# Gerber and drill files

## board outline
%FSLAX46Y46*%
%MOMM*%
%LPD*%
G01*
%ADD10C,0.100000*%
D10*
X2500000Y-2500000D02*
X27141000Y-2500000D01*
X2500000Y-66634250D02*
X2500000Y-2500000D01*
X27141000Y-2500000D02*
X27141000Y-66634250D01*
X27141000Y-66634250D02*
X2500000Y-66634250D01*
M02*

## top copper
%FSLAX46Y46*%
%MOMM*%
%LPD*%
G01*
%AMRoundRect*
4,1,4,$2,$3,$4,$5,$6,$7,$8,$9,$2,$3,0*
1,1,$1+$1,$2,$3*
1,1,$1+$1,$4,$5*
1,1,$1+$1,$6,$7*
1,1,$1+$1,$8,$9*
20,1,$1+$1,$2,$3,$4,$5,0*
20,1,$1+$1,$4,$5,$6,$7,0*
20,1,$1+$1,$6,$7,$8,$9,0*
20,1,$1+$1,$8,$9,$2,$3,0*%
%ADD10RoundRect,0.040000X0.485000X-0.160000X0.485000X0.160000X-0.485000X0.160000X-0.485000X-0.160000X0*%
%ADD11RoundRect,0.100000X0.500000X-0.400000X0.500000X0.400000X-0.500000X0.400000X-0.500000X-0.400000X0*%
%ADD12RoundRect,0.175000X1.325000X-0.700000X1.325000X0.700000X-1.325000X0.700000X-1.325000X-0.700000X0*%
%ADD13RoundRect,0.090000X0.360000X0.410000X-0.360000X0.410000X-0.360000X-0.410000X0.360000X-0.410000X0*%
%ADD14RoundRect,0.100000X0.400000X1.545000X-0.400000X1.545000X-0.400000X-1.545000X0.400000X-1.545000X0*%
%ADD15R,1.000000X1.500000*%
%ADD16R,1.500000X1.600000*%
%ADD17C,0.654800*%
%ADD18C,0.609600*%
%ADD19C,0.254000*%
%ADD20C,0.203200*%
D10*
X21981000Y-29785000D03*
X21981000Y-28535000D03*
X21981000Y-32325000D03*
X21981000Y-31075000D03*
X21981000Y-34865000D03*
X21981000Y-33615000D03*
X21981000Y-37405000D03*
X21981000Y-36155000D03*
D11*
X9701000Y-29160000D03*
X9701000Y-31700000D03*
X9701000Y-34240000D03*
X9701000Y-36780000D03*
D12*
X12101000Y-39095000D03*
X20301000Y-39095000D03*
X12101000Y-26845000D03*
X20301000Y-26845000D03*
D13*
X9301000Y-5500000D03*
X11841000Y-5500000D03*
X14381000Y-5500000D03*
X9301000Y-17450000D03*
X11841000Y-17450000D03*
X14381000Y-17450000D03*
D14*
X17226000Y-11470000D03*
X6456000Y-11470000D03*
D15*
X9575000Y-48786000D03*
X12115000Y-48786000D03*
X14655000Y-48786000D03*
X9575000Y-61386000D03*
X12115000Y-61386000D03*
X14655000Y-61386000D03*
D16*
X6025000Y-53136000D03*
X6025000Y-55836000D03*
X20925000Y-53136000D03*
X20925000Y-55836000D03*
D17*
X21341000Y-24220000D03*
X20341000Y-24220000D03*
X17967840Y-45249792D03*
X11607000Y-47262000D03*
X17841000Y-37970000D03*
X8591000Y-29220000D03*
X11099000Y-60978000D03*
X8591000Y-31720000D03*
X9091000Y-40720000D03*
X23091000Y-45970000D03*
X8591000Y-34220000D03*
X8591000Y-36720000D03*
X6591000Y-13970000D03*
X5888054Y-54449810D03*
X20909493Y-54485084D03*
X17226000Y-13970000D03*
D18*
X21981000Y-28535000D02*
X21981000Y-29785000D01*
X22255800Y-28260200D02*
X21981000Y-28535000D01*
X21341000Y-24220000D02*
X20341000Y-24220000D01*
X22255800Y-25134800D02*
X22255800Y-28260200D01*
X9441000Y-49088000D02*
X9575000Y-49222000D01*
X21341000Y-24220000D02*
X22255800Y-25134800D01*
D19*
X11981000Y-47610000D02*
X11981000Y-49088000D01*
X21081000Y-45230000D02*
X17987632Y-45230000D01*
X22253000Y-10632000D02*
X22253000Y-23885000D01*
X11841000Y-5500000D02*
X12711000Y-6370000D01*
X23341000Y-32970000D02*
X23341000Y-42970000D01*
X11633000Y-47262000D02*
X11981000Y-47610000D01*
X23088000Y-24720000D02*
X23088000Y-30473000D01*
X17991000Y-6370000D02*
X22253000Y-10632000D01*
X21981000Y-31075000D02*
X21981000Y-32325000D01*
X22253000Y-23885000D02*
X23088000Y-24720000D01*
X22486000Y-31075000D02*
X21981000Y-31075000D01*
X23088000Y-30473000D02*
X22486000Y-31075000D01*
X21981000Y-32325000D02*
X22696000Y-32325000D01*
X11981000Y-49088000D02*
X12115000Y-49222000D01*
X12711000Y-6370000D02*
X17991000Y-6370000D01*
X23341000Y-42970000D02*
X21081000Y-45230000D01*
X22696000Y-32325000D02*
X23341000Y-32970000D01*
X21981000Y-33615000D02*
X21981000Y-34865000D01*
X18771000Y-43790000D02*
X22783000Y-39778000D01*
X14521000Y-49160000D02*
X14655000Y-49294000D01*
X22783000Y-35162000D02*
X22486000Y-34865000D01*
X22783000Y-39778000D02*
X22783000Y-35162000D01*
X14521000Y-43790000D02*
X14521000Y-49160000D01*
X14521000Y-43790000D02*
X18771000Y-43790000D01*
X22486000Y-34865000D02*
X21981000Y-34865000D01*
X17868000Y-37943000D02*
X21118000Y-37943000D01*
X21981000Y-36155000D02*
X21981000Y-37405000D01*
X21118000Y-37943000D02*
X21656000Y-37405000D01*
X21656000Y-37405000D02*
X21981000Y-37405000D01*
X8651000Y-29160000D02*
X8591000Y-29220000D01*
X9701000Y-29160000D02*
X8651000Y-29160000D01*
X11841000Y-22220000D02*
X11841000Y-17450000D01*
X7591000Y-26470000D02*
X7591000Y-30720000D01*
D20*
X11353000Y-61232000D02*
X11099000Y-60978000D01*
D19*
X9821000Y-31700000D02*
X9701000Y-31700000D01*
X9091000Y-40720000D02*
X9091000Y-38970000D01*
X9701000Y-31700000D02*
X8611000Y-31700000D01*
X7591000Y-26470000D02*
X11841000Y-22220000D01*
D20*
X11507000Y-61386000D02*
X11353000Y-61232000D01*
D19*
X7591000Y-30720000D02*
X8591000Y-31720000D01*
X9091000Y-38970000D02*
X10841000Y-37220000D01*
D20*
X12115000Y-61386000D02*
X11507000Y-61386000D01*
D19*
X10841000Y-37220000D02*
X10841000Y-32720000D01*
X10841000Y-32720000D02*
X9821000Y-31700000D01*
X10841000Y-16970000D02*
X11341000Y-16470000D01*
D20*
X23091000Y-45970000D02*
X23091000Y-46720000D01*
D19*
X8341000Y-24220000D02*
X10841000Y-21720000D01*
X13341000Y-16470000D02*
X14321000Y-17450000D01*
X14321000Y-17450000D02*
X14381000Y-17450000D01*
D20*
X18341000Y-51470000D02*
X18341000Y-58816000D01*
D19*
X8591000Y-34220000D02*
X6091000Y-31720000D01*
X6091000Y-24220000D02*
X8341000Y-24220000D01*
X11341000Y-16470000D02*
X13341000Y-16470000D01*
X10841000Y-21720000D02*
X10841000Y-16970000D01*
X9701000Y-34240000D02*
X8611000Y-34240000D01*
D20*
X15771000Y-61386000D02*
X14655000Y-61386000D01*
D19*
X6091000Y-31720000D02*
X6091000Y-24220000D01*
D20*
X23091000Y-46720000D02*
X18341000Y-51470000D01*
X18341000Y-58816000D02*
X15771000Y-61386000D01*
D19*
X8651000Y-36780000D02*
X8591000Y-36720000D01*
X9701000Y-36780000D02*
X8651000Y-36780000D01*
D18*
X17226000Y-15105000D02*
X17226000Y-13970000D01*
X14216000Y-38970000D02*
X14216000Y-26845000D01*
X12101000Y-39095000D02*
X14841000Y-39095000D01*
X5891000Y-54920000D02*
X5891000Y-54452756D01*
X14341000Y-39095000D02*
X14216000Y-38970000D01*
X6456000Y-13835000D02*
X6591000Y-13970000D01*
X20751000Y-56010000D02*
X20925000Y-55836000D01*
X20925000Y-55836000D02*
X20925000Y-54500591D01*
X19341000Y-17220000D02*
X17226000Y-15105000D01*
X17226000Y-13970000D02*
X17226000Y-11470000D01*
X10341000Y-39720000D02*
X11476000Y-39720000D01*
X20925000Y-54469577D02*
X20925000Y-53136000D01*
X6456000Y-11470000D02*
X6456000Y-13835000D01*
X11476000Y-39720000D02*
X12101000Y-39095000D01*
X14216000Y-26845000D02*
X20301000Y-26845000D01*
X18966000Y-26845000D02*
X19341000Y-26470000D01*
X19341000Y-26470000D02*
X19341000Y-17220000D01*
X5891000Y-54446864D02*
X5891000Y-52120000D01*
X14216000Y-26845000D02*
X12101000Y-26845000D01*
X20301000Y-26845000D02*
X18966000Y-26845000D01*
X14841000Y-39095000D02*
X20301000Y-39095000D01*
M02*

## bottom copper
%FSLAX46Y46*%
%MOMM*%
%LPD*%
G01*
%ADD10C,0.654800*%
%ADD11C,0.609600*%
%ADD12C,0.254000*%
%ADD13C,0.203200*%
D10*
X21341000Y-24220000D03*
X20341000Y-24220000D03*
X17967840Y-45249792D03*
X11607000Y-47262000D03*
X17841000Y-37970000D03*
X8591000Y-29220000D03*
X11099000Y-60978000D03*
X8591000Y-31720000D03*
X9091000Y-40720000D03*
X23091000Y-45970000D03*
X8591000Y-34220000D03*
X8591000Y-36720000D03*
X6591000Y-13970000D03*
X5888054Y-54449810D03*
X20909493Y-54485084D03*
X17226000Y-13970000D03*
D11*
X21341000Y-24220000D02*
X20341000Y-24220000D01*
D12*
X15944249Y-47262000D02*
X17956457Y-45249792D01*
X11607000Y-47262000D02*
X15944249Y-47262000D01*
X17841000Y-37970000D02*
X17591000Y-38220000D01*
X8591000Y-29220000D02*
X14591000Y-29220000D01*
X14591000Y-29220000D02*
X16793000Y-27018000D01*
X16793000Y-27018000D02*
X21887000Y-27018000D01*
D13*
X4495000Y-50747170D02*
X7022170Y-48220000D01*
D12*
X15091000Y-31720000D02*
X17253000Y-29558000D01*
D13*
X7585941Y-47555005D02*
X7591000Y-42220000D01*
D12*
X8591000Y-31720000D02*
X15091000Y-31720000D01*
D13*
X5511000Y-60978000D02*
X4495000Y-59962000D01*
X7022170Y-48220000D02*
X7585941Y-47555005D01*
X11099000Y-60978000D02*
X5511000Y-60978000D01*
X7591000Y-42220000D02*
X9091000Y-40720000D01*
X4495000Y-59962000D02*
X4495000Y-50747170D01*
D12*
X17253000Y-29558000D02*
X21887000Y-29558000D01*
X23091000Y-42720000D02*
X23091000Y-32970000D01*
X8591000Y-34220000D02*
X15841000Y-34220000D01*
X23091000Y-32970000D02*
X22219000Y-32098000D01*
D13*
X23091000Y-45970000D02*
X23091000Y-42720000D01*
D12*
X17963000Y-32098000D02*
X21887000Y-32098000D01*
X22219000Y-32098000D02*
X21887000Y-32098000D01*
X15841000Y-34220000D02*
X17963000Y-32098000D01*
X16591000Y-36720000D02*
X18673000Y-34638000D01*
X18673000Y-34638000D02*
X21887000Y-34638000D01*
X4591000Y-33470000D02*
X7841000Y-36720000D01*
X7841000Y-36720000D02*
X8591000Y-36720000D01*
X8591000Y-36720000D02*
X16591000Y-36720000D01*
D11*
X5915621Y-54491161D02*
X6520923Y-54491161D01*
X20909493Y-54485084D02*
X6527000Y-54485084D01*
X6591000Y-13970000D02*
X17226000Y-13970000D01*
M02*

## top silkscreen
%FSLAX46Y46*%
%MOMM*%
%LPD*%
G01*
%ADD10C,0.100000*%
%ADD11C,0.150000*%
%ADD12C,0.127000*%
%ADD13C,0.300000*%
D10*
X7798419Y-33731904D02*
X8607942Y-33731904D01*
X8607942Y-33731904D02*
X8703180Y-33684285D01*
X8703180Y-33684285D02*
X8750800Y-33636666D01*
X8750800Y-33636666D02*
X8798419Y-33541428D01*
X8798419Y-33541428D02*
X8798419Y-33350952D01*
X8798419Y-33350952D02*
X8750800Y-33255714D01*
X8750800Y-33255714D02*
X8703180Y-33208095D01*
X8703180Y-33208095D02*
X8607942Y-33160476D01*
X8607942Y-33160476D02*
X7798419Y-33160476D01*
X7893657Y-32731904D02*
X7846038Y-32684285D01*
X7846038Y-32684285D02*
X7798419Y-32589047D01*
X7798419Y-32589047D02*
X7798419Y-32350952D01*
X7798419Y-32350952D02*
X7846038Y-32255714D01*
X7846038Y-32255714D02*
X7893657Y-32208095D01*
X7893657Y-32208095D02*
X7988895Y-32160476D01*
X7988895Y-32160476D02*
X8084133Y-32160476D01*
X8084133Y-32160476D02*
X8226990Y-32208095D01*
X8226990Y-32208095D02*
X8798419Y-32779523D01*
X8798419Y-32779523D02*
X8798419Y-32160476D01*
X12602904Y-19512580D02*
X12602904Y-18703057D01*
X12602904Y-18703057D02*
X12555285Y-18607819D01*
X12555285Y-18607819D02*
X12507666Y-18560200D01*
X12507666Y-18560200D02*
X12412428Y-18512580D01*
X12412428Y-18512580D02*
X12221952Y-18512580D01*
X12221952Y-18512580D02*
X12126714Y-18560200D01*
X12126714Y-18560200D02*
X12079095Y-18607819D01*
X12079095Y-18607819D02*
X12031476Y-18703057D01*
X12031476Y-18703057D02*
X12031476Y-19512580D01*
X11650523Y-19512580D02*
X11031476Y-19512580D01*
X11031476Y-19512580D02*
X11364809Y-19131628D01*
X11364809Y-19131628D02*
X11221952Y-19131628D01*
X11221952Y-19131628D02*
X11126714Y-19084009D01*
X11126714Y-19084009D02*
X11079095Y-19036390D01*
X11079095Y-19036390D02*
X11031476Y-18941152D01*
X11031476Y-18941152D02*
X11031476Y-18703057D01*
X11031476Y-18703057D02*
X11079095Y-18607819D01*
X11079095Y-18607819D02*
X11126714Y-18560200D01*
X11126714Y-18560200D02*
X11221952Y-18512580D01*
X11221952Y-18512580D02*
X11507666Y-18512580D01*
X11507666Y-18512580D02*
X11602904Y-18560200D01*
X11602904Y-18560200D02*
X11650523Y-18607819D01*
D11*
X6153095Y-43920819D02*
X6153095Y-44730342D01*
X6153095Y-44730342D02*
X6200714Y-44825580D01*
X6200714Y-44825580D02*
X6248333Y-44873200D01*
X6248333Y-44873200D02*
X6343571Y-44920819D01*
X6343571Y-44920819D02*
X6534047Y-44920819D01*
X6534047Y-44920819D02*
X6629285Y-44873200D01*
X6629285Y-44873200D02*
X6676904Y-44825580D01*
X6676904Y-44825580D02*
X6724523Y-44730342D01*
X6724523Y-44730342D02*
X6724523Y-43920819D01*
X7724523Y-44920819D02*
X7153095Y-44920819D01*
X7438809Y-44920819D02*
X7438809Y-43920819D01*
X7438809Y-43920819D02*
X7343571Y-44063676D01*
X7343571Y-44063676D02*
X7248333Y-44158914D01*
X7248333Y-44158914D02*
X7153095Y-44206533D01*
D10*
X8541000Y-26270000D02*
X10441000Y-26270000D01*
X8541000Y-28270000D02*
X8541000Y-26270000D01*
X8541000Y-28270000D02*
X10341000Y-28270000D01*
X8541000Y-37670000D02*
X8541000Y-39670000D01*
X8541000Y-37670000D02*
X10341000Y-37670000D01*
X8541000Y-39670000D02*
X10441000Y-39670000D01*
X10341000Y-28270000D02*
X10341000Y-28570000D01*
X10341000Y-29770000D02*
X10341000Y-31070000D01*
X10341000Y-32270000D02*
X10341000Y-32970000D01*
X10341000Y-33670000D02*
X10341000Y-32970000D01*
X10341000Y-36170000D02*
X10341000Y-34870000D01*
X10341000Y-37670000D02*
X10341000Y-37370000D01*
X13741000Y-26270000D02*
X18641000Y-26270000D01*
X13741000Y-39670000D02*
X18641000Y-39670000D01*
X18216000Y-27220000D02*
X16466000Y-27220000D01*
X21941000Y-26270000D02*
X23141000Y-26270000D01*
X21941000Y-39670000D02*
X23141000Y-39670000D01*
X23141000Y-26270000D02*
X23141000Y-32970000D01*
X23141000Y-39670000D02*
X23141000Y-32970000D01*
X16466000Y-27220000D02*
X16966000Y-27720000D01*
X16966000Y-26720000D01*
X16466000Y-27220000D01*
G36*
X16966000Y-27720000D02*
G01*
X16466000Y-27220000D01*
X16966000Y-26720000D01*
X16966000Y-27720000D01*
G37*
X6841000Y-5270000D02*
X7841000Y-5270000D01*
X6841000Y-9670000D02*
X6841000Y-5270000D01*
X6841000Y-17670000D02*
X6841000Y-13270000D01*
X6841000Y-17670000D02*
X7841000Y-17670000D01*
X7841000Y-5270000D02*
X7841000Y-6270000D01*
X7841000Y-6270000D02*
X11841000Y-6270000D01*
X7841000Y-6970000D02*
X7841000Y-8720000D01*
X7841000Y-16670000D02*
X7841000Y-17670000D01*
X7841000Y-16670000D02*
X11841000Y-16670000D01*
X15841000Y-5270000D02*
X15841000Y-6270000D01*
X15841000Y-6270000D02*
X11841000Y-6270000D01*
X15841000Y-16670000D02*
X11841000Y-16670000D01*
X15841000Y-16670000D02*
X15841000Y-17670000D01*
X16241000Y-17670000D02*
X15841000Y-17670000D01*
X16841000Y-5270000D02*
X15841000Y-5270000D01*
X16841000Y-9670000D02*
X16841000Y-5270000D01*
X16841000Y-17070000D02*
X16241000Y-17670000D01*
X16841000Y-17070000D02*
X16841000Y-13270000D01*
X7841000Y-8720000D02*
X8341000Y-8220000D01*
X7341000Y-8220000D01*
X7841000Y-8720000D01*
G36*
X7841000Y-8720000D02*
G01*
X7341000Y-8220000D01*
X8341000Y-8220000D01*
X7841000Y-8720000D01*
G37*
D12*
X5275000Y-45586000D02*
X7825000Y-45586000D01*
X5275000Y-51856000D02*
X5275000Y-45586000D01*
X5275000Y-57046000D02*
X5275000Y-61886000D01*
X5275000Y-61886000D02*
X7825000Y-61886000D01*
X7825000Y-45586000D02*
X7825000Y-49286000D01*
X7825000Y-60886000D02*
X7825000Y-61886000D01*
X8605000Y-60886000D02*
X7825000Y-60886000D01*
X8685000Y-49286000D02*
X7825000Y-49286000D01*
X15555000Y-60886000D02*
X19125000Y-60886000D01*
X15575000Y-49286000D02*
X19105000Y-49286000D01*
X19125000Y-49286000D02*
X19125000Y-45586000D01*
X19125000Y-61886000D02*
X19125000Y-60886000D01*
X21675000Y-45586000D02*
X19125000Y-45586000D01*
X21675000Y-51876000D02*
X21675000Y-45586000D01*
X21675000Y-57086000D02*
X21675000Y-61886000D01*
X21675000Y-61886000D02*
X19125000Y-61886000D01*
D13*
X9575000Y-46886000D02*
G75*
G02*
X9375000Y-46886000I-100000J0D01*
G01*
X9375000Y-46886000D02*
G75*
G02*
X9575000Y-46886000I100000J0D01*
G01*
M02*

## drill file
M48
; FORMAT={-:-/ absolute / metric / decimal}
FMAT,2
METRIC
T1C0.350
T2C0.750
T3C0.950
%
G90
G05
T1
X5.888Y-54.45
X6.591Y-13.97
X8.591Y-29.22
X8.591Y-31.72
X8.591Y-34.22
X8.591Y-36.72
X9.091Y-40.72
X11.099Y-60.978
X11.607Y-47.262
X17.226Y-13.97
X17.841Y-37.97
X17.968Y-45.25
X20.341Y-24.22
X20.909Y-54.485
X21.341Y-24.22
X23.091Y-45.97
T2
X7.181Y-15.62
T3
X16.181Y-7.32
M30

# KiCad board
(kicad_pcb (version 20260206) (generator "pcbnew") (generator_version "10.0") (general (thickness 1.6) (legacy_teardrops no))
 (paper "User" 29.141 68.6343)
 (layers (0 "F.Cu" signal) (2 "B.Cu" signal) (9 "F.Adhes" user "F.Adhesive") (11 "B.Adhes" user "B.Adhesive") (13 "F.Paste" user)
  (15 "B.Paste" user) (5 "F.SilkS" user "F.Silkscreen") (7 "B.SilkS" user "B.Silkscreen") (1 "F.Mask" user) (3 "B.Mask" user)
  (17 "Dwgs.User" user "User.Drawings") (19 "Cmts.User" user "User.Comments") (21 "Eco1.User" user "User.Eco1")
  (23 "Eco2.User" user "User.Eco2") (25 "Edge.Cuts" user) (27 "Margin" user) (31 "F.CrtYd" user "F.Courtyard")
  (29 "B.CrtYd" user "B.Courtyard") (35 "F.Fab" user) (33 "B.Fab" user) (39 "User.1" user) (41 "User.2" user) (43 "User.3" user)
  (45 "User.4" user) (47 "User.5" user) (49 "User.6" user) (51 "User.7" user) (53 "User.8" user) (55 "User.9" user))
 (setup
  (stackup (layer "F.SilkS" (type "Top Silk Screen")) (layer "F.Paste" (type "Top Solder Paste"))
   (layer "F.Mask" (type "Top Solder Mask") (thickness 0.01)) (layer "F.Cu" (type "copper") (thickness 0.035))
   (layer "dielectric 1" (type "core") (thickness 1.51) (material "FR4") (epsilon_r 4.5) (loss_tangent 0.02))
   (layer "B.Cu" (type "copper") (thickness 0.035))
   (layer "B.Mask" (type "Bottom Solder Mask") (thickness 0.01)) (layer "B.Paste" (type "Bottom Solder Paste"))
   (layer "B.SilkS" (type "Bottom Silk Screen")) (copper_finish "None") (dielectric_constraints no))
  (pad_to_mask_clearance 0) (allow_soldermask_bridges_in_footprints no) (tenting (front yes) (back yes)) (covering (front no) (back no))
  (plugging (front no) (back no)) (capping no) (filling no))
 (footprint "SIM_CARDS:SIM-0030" (layer "F.Cu") (at 15.841 32.97 90)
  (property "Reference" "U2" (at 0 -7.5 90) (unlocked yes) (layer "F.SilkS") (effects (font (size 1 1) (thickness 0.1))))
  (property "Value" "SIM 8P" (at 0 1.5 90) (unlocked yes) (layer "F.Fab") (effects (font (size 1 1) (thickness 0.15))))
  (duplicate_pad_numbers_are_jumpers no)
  (fp_line (start 6.7 -7.3) (end 6.7 -5.4) (stroke (width 0.1) (type default)) (layer "F.SilkS"))
  (fp_line (start 4.7 -7.3) (end 6.7 -7.3) (stroke (width 0.1) (type default)) (layer "F.SilkS"))
  (fp_line (start 4.7 -7.3) (end 4.7 -5.5) (stroke (width 0.1) (type default)) (layer "F.SilkS"))
  (fp_line (start -4.7 -7.3) (end -6.7 -7.3) (stroke (width 0.1) (type default)) (layer "F.SilkS"))
  (fp_line (start -4.7 -7.3) (end -4.7 -5.5) (stroke (width 0.1) (type default)) (layer "F.SilkS"))
  (fp_line (start -6.7 -7.3) (end -6.7 -5.4) (stroke (width 0.1) (type default)) (layer "F.SilkS"))
  (fp_line (start 4.7 -5.5) (end 4.4 -5.5) (stroke (width 0.1) (type default)) (layer "F.SilkS"))
  (fp_line (start 3.2 -5.5) (end 1.9 -5.5) (stroke (width 0.1) (type default)) (layer "F.SilkS"))
  (fp_line (start 0.7 -5.5) (end 0 -5.5) (stroke (width 0.1) (type default)) (layer "F.SilkS"))
  (fp_line (start -0.7 -5.5) (end 0 -5.5) (stroke (width 0.1) (type default)) (layer "F.SilkS"))
  (fp_line (start -3.2 -5.5) (end -1.9 -5.5) (stroke (width 0.1) (type default)) (layer "F.SilkS"))
  (fp_line (start -4.7 -5.5) (end -4.4 -5.5) (stroke (width 0.1) (type default)) (layer "F.SilkS"))
  (fp_line (start 6.7 -2.1) (end 6.7 2.8) (stroke (width 0.1) (type default)) (layer "F.SilkS"))
  (fp_line (start -6.7 -2.1) (end -6.7 2.8) (stroke (width 0.1) (type default)) (layer "F.SilkS"))
  (fp_line (start 5.75 2.375) (end 5.75 0.625) (stroke (width 0.1) (type default)) (layer "F.SilkS"))
  (fp_line (start 6.7 6.1) (end 6.7 7.3) (stroke (width 0.1) (type default)) (layer "F.SilkS"))
  (fp_line (start -6.7 6.1) (end -6.7 7.3) (stroke (width 0.1) (type default)) (layer "F.SilkS"))
  (fp_line (start 6.7 7.3) (end 0 7.3) (stroke (width 0.1) (type default)) (layer "F.SilkS"))
  (fp_line (start -6.7 7.3) (end 0 7.3) (stroke (width 0.1) (type default)) (layer "F.SilkS"))
  (fp_poly (pts (xy 5.75 0.625) (xy 5.25 1.125) (xy 6.25 1.125)) (stroke (width 0.1) (type solid)) (fill yes) (layer "F.SilkS"))
  (pad "C1" smd roundrect (at 3.185 6.14 90) (size 0.4 1.05) (layers "F.Cu" "F.Mask" "F.Paste") (roundrect_rratio 0.1) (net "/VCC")
   (thermal_bridge_angle 45))
  (pad "C1" smd roundrect (at 4.435 6.14 90) (size 0.4 1.05) (layers "F.Cu" "F.Mask" "F.Paste") (roundrect_rratio 0.1) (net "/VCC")
   (thermal_bridge_angle 45))
  (pad "C2" smd roundrect (at 0.645 6.14 90) (size 0.4 1.05) (layers "F.Cu" "F.Mask" "F.Paste") (roundrect_rratio 0.1) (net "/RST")
   (thermal_bridge_angle 45))
  (pad "C2" smd roundrect (at 1.895 6.14 90) (size 0.4 1.05) (layers "F.Cu" "F.Mask" "F.Paste") (roundrect_rratio 0.1) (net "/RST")
   (thermal_bridge_angle 45))
  (pad "C3" smd roundrect (at -1.895 6.14 90) (size 0.4 1.05) (layers "F.Cu" "F.Mask" "F.Paste") (roundrect_rratio 0.1) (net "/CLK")
   (thermal_bridge_angle 45))
  (pad "C3" smd roundrect (at -0.645 6.14 90) (size 0.4 1.05) (layers "F.Cu" "F.Mask" "F.Paste") (roundrect_rratio 0.1) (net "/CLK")
   (thermal_bridge_angle 45))
  (pad "C4" smd roundrect (at -4.435 6.14 90) (size 0.4 1.05) (layers "F.Cu" "F.Mask" "F.Paste") (roundrect_rratio 0.1) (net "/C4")
   (thermal_bridge_angle 45))
  (pad "C4" smd roundrect (at -3.185 6.14 90) (size 0.4 1.05) (layers "F.Cu" "F.Mask" "F.Paste") (roundrect_rratio 0.1) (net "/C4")
   (thermal_bridge_angle 45))
  (pad "C5" smd roundrect (at 3.81 -6.14 90) (size 1 1.2) (layers "F.Cu" "F.Mask" "F.Paste") (roundrect_rratio 0.1) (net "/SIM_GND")
   (thermal_bridge_angle 45))
  (pad "C6" smd roundrect (at 1.27 -6.14 90) (size 1 1.2) (layers "F.Cu" "F.Mask" "F.Paste") (roundrect_rratio 0.1) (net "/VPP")
   (thermal_bridge_angle 45))
  (pad "C7" smd roundrect (at -1.27 -6.14 90) (size 1 1.2) (layers "F.Cu" "F.Mask" "F.Paste") (roundrect_rratio 0.1) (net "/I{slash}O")
   (thermal_bridge_angle 45))
  (pad "C8" smd roundrect (at -3.81 -6.14 90) (size 1 1.2) (layers "F.Cu" "F.Mask" "F.Paste") (roundrect_rratio 0.1) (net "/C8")
   (thermal_bridge_angle 45))
  (pad "SH" smd roundrect (at -6.125 -3.74 90) (size 1.75 3) (layers "F.Cu" "F.Mask" "F.Paste") (roundrect_rratio 0.1) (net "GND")
   (thermal_bridge_angle 45))
  (pad "SH" smd roundrect (at -6.125 4.46 90) (size 1.75 3) (layers "F.Cu" "F.Mask" "F.Paste") (roundrect_rratio 0.1) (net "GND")
   (thermal_bridge_angle 45))
  (pad "SH" smd roundrect (at 6.125 -3.74 90) (size 1.75 3) (layers "F.Cu" "F.Mask" "F.Paste") (roundrect_rratio 0.1) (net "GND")
   (thermal_bridge_angle 45))
  (pad "SH" smd roundrect (at 6.125 4.46 90) (size 1.75 3) (layers "F.Cu" "F.Mask" "F.Paste") (roundrect_rratio 0.1) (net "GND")
   (thermal_bridge_angle 45))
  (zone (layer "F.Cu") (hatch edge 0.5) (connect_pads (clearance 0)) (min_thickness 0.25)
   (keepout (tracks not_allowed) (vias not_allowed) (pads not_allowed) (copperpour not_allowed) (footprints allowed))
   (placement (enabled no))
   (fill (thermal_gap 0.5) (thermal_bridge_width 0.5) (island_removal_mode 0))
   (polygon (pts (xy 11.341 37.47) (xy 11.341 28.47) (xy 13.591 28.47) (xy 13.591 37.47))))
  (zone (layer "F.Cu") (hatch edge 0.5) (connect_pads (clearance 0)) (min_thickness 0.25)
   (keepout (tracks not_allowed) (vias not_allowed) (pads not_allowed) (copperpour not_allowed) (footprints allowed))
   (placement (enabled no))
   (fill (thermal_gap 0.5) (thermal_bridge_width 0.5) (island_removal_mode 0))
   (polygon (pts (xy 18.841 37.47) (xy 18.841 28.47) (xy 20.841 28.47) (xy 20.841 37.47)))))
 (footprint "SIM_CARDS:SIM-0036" (layer "F.Cu") (at 11.841 11.47 180)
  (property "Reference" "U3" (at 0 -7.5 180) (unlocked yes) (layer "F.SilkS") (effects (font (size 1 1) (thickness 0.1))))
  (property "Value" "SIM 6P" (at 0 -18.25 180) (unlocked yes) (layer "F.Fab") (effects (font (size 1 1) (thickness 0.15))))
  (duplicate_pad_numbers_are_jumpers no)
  (fp_line (start 5 6.2) (end 4 6.2) (stroke (width 0.1) (type default)) (layer "F.SilkS"))
  (fp_line (start 5 1.8) (end 5 6.2) (stroke (width 0.1) (type default)) (layer "F.SilkS"))
  (fp_line (start 5 -6.2) (end 5 -1.8) (stroke (width 0.1) (type default)) (layer "F.SilkS"))
  (fp_line (start 5 -6.2) (end 4 -6.2) (stroke (width 0.1) (type default)) (layer "F.SilkS"))
  (fp_line (start 4 6.2) (end 4 5.2) (stroke (width 0.1) (type default)) (layer "F.SilkS"))
  (fp_line (start 4 5.2) (end 0 5.2) (stroke (width 0.1) (type default)) (layer "F.SilkS"))
  (fp_line (start 4 4.5) (end 4 2.75) (stroke (width 0.1) (type default)) (layer "F.SilkS"))
  (fp_line (start 4 -5.2) (end 4 -6.2) (stroke (width 0.1) (type default)) (layer "F.SilkS"))
  (fp_line (start 4 -5.2) (end 0 -5.2) (stroke (width 0.1) (type default)) (layer "F.SilkS"))
  (fp_line (start -4 6.2) (end -4 5.2) (stroke (width 0.1) (type default)) (layer "F.SilkS"))
  (fp_line (start -4 5.2) (end 0 5.2) (stroke (width 0.1) (type default)) (layer "F.SilkS"))
  (fp_line (start -4 -5.2) (end 0 -5.2) (stroke (width 0.1) (type default)) (layer "F.SilkS"))
  (fp_line (start -4 -5.2) (end -4 -6.2) (stroke (width 0.1) (type default)) (layer "F.SilkS"))
  (fp_line (start -4.4 -6.2) (end -4 -6.2) (stroke (width 0.1) (type default)) (layer "F.SilkS"))
  (fp_line (start -5 6.2) (end -4 6.2) (stroke (width 0.1) (type default)) (layer "F.SilkS"))
  (fp_line (start -5 1.8) (end -5 6.2) (stroke (width 0.1) (type default)) (layer "F.SilkS"))
  (fp_line (start -5 -5.6) (end -4.4 -6.2) (stroke (width 0.1) (type default)) (layer "F.SilkS"))
  (fp_line (start -5 -5.6) (end -5 -1.8) (stroke (width 0.1) (type default)) (layer "F.SilkS"))
  (fp_poly (pts (xy 4 2.75) (xy 3.5 3.25) (xy 4.5 3.25)) (stroke (width 0.1) (type solid)) (fill yes) (layer "F.SilkS"))
  (pad "" np_thru_hole circle (at -4.34 4.15 180) (size 0.95 0.95) (drill 0.95) (layers "*.Cu" "*.Mask"))
  (pad "" np_thru_hole circle (at 4.66 -4.15 180) (size 0.75 0.75) (drill 0.75) (layers "*.Cu" "*.Mask"))
  (pad "C1" smd roundrect (at 2.54 5.97 180) (size 0.9 1) (layers "F.Cu" "F.Mask" "F.Paste") (roundrect_rratio 0.1) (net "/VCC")
   (thermal_bridge_angle 45))
  (pad "C2" smd roundrect (at 0 5.97 180) (size 0.9 1) (layers "F.Cu" "F.Mask" "F.Paste") (roundrect_rratio 0.1) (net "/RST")
   (thermal_bridge_angle 45))
  (pad "C3" smd roundrect (at -2.54 5.97 180) (size 0.9 1) (layers "F.Cu" "F.Mask" "F.Paste") (roundrect_rratio 0.1) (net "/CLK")
   (thermal_bridge_angle 45))
  (pad "C5" smd roundrect (at 2.54 -5.98 180) (size 0.9 1) (layers "F.Cu" "F.Mask" "F.Paste") (roundrect_rratio 0.1) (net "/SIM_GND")
   (thermal_bridge_angle 45))
  (pad "C6" smd roundrect (at 0 -5.98 180) (size 0.9 1) (layers "F.Cu" "F.Mask" "F.Paste") (roundrect_rratio 0.1) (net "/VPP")
   (thermal_bridge_angle 45))
  (pad "C7" smd roundrect (at -2.54 -5.98 180) (size 0.9 1) (layers "F.Cu" "F.Mask" "F.Paste") (roundrect_rratio 0.1) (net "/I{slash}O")
   (thermal_bridge_angle 45))
  (pad "SH" smd roundrect (at -5.385 0 180) (size 1 3.29) (layers "F.Cu" "F.Mask" "F.Paste") (roundrect_rratio 0.1) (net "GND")
   (thermal_bridge_angle 45))
  (pad "SH" smd roundrect (at 5.385 0 180) (size 1 3.29) (layers "F.Cu" "F.Mask" "F.Paste") (roundrect_rratio 0.1) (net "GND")
   (thermal_bridge_angle 45)))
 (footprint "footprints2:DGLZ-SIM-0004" (layer "F.Cu") (at 13.315 54.446)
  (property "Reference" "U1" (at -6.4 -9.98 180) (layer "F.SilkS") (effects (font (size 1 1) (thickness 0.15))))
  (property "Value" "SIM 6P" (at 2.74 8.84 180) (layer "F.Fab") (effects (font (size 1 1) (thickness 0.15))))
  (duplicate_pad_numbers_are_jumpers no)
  (fp_line (start -8.04 -8.86) (end -5.49 -8.86) (stroke (width 0.127) (type solid)) (layer "F.SilkS"))
  (fp_line (start -8.04 -2.59) (end -8.04 -8.86) (stroke (width 0.127) (type solid)) (layer "F.SilkS"))
  (fp_line (start -8.04 2.6) (end -8.04 7.44) (stroke (width 0.127) (type solid)) (layer "F.SilkS"))
  (fp_line (start -8.04 7.44) (end -5.49 7.44) (stroke (width 0.127) (type solid)) (layer "F.SilkS"))
  (fp_line (start -5.49 -8.86) (end -5.49 -5.16) (stroke (width 0.127) (type solid)) (layer "F.SilkS"))
  (fp_line (start -5.49 6.44) (end -5.49 7.44) (stroke (width 0.127) (type solid)) (layer "F.SilkS"))
  (fp_line (start -4.71 6.44) (end -5.49 6.44) (stroke (width 0.127) (type solid)) (layer "F.SilkS"))
  (fp_line (start -4.63 -5.16) (end -5.49 -5.16) (stroke (width 0.127) (type solid)) (layer "F.SilkS"))
  (fp_line (start 2.24 6.44) (end 5.81 6.44) (stroke (width 0.127) (type solid)) (layer "F.SilkS"))
  (fp_line (start 2.26 -5.16) (end 5.79 -5.16) (stroke (width 0.127) (type solid)) (layer "F.SilkS"))
  (fp_line (start 5.81 -5.16) (end 5.81 -8.86) (stroke (width 0.127) (type solid)) (layer "F.SilkS"))
  (fp_line (start 5.81 7.44) (end 5.81 6.44) (stroke (width 0.127) (type solid)) (layer "F.SilkS"))
  (fp_line (start 8.36 -8.86) (end 5.81 -8.86) (stroke (width 0.127) (type solid)) (layer "F.SilkS"))
  (fp_line (start 8.36 -2.57) (end 8.36 -8.86) (stroke (width 0.127) (type solid)) (layer "F.SilkS"))
  (fp_line (start 8.36 2.64) (end 8.36 7.44) (stroke (width 0.127) (type solid)) (layer "F.SilkS"))
  (fp_line (start 8.36 7.44) (end 5.81 7.44) (stroke (width 0.127) (type solid)) (layer "F.SilkS"))
  (fp_circle (center -3.84 -7.56) (end -3.74 -7.56) (stroke (width 0.3) (type solid)) (fill no) (layer "F.SilkS"))
  (pad "C1" smd rect (at -3.74 -5.66 180) (size 1 1.5) (layers "F.Cu" "F.Mask" "F.Paste") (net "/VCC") (solder_mask_margin 0.102))
  (pad "C2" smd rect (at -1.2 -5.66 180) (size 1 1.5) (layers "F.Cu" "F.Mask" "F.Paste") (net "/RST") (solder_mask_margin 0.102))
  (pad "C3" smd rect (at 1.34 -5.66 180) (size 1 1.5) (layers "F.Cu" "F.Mask" "F.Paste") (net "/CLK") (solder_mask_margin 0.102))
  (pad "C5" smd rect (at -3.74 6.94 180) (size 1 1.5) (layers "F.Cu" "F.Mask" "F.Paste") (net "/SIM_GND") (solder_mask_margin 0.102))
  (pad "C6" smd rect (at -1.2 6.94 180) (size 1 1.5) (layers "F.Cu" "F.Mask" "F.Paste") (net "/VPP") (solder_mask_margin 0.102))
  (pad "C7" smd rect (at 1.34 6.94 180) (size 1 1.5) (layers "F.Cu" "F.Mask" "F.Paste") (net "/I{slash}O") (solder_mask_margin 0.102))
  (pad "SH" smd rect (at -7.29 -1.31 180) (size 1.5 1.6) (layers "F.Cu" "F.Mask" "F.Paste") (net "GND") (solder_mask_margin 0.102))
  (pad "SH" smd rect (at -7.29 1.39 180) (size 1.5 1.6) (layers "F.Cu" "F.Mask" "F.Paste") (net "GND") (solder_mask_margin 0.102))
  (pad "SH" smd rect (at 7.61 -1.31 180) (size 1.5 1.6) (layers "F.Cu" "F.Mask" "F.Paste") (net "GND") (solder_mask_margin 0.102))
  (pad "SH" smd rect (at 7.61 1.39 180) (size 1.5 1.6) (layers "F.Cu" "F.Mask" "F.Paste") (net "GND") (solder_mask_margin 0.102))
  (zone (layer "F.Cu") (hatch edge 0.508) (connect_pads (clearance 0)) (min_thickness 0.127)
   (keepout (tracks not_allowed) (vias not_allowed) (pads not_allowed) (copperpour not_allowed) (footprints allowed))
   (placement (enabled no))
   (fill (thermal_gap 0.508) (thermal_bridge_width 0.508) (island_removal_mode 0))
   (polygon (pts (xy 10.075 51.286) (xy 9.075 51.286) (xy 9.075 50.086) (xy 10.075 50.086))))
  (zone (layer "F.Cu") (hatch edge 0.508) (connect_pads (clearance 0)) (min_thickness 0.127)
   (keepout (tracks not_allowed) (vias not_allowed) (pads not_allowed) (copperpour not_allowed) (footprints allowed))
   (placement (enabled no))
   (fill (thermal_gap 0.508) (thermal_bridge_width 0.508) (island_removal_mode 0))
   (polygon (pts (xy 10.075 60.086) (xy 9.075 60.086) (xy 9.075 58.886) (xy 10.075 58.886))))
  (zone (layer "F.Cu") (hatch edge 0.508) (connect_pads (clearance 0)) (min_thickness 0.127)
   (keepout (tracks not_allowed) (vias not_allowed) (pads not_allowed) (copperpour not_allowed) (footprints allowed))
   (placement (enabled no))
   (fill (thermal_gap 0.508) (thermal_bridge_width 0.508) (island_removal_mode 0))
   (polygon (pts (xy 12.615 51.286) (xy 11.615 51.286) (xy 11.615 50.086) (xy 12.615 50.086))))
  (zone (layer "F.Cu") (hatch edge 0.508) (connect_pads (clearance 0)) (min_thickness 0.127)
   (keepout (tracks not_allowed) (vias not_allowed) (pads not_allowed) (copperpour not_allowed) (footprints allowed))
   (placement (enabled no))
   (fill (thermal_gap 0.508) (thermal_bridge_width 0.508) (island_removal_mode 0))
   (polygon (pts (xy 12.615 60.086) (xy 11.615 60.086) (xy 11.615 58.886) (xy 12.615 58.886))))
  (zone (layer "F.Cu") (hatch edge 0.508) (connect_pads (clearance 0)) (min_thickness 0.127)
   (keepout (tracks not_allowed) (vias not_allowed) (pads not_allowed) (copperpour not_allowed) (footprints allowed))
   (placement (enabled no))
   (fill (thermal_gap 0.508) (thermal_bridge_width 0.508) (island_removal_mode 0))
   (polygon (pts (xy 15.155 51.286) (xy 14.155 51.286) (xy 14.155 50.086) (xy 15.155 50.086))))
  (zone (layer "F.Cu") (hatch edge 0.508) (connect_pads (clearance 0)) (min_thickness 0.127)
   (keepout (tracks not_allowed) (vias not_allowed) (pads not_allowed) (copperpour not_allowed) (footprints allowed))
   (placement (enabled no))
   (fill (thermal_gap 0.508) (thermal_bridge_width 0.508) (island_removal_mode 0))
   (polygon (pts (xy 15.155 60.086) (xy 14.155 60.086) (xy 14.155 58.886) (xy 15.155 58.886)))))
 (gr_line (start 2.5 2.5) (end 27.141 2.5) (stroke (width 0.1) (type default)) (layer "Edge.Cuts"))
 (gr_line (start 2.5 66.63425) (end 2.5 2.5) (stroke (width 0.1) (type default)) (layer "Edge.Cuts"))
 (gr_line (start 27.141 2.5) (end 27.141 66.63425) (stroke (width 0.1) (type default)) (layer "Edge.Cuts"))
 (gr_line (start 27.141 66.63425) (end 2.5 66.63425) (stroke (width 0.1) (type default)) (layer "Edge.Cuts"))
 (segment (start 21.981 28.535) (end 21.981 29.785) (width 0.6096) (layer "F.Cu") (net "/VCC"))
 (segment (start 22.2558 28.2602) (end 21.981 28.535) (width 0.6096) (layer "F.Cu") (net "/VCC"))
 (segment (start 21.341 24.22) (end 20.341 24.22) (width 0.6096) (layer "F.Cu") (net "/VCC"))
 (segment (start 22.2558 25.1348) (end 22.2558 28.2602) (width 0.6096) (layer "F.Cu") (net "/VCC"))
 (segment (start 9.441 49.088) (end 9.575 49.222) (width 0.6096) (layer "F.Cu") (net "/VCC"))
 (segment (start 21.341 24.22) (end 22.2558 25.1348) (width 0.6096) (layer "F.Cu") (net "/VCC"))
 (via (at 21.341 24.22) (size 0.6548) (drill 0.35) (layers "F.Cu" "B.Cu") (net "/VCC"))
 (via (at 20.341 24.22) (size 0.6548) (drill 0.35) (layers "F.Cu" "B.Cu") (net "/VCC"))
 (segment (start 21.341 24.22) (end 20.341 24.22) (width 0.6096) (layer "B.Cu") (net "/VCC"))
 (segment (start 11.981 47.61) (end 11.981 49.088) (width 0.254) (layer "F.Cu") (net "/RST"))
 (segment (start 21.081 45.23) (end 17.987632 45.23) (width 0.254) (layer "F.Cu") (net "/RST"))
 (segment (start 22.253 10.632) (end 22.253 23.885) (width 0.254) (layer "F.Cu") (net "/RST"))
 (segment (start 11.841 5.5) (end 12.711 6.37) (width 0.254) (layer "F.Cu") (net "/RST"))
 (segment (start 23.341 32.97) (end 23.341 42.97) (width 0.254) (layer "F.Cu") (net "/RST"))
 (segment (start 11.633 47.262) (end 11.981 47.61) (width 0.254) (layer "F.Cu") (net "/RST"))
 (segment (start 23.088 24.72) (end 23.088 30.473) (width 0.254) (layer "F.Cu") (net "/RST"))
 (segment (start 17.991 6.37) (end 22.253 10.632) (width 0.254) (layer "F.Cu") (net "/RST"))
 (segment (start 21.981 31.075) (end 21.981 32.325) (width 0.254) (layer "F.Cu") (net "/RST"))
 (segment (start 22.253 23.885) (end 23.088 24.72) (width 0.254) (layer "F.Cu") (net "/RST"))
 (segment (start 22.486 31.075) (end 21.981 31.075) (width 0.254) (layer "F.Cu") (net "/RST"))
 (segment (start 23.088 30.473) (end 22.486 31.075) (width 0.254) (layer "F.Cu") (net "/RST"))
 (segment (start 21.981 32.325) (end 22.696 32.325) (width 0.254) (layer "F.Cu") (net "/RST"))
 (segment (start 11.981 49.088) (end 12.115 49.222) (width 0.254) (layer "F.Cu") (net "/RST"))
 (segment (start 12.711 6.37) (end 17.991 6.37) (width 0.254) (layer "F.Cu") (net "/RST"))
 (segment (start 23.341 42.97) (end 21.081 45.23) (width 0.254) (layer "F.Cu") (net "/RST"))
 (segment (start 22.696 32.325) (end 23.341 32.97) (width 0.254) (layer "F.Cu") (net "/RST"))
 (via (at 17.96784 45.249792) (size 0.6548) (drill 0.35) (layers "F.Cu" "B.Cu") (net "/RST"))
 (via (at 11.607 47.262) (size 0.6548) (drill 0.35) (layers "F.Cu" "B.Cu") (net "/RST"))
 (segment (start 15.944249 47.262) (end 17.956457 45.249792) (width 0.254) (layer "B.Cu") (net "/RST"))
 (segment (start 11.607 47.262) (end 15.944249 47.262) (width 0.254) (layer "B.Cu") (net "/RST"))
 (segment (start 21.981 33.615) (end 21.981 34.865) (width 0.254) (layer "F.Cu") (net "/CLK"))
 (segment (start 18.771 43.79) (end 22.783 39.778) (width 0.254) (layer "F.Cu") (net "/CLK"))
 (segment (start 14.521 49.16) (end 14.655 49.294) (width 0.254) (layer "F.Cu") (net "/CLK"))
 (segment (start 22.783 35.162) (end 22.486 34.865) (width 0.254) (layer "F.Cu") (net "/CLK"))
 (segment (start 22.783 39.778) (end 22.783 35.162) (width 0.254) (layer "F.Cu") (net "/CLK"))
 (segment (start 14.521 43.79) (end 14.521 49.16) (width 0.254) (layer "F.Cu") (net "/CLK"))
 (segment (start 14.521 43.79) (end 18.771 43.79) (width 0.254) (layer "F.Cu") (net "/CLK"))
 (segment (start 22.486 34.865) (end 21.981 34.865) (width 0.254) (layer "F.Cu") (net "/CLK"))
 (segment (start 17.868 37.943) (end 21.118 37.943) (width 0.254) (layer "F.Cu") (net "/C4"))
 (segment (start 21.981 36.155) (end 21.981 37.405) (width 0.254) (layer "F.Cu") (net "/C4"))
 (segment (start 21.118 37.943) (end 21.656 37.405) (width 0.254) (layer "F.Cu") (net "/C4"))
 (segment (start 21.656 37.405) (end 21.981 37.405) (width 0.254) (layer "F.Cu") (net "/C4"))
 (via (at 17.841 37.97) (size 0.6548) (drill 0.35) (layers "F.Cu" "B.Cu") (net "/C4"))
 (segment (start 17.841 37.97) (end 17.591 38.22) (width 0.254) (layer "B.Cu") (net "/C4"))
 (segment (start 8.651 29.16) (end 8.591 29.22) (width 0.254) (layer "F.Cu") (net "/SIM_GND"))
 (segment (start 9.701 29.16) (end 8.651 29.16) (width 0.254) (layer "F.Cu") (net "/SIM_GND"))
 (via (at 8.591 29.22) (size 0.6548) (drill 0.35) (layers "F.Cu" "B.Cu") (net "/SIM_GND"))
 (segment (start 8.591 29.22) (end 14.591 29.22) (width 0.254) (layer "B.Cu") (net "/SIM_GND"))
 (segment (start 14.591 29.22) (end 16.793 27.018) (width 0.254) (layer "B.Cu") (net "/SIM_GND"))
 (segment (start 16.793 27.018) (end 21.887 27.018) (width 0.254) (layer "B.Cu") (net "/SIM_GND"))
 (segment (start 11.841 22.22) (end 11.841 17.45) (width 0.254) (layer "F.Cu") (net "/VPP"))
 (segment (start 7.591 26.47) (end 7.591 30.72) (width 0.254) (layer "F.Cu") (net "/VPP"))
 (segment (start 11.353 61.232) (end 11.099 60.978) (width 0.2032) (layer "F.Cu") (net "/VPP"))
 (segment (start 9.821 31.7) (end 9.701 31.7) (width 0.254) (layer "F.Cu") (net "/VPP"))
 (segment (start 9.091 40.72) (end 9.091 38.97) (width 0.254) (layer "F.Cu") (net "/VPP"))
 (segment (start 9.701 31.7) (end 8.611 31.7) (width 0.254) (layer "F.Cu") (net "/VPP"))
 (segment (start 7.591 26.47) (end 11.841 22.22) (width 0.254) (layer "F.Cu") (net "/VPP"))
 (segment (start 11.507 61.386) (end 11.353 61.232) (width 0.2032) (layer "F.Cu") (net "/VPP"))
 (segment (start 7.591 30.72) (end 8.591 31.72) (width 0.254) (layer "F.Cu") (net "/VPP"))
 (segment (start 9.091 38.97) (end 10.841 37.22) (width 0.254) (layer "F.Cu") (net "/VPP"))
 (segment (start 12.115 61.386) (end 11.507 61.386) (width 0.2032) (layer "F.Cu") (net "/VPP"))
 (segment (start 10.841 37.22) (end 10.841 32.72) (width 0.254) (layer "F.Cu") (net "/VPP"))
 (segment (start 10.841 32.72) (end 9.821 31.7) (width 0.254) (layer "F.Cu") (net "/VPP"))
 (via (at 11.099 60.978) (size 0.6548) (drill 0.35) (layers "F.Cu" "B.Cu") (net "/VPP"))
 (via (at 8.591 31.72) (size 0.6548) (drill 0.35) (layers "F.Cu" "B.Cu") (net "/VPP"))
 (via (at 9.091 40.72) (size 0.6548) (drill 0.35) (layers "F.Cu" "B.Cu") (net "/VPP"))
 (segment (start 4.495 50.74717) (end 7.02217 48.22) (width 0.2032) (layer "B.Cu") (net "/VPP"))
 (segment (start 15.091 31.72) (end 17.253 29.558) (width 0.254) (layer "B.Cu") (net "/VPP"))
 (segment (start 7.585941 47.555005) (end 7.591 42.22) (width 0.2032) (layer "B.Cu") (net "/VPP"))
 (segment (start 8.591 31.72) (end 15.091 31.72) (width 0.254) (layer "B.Cu") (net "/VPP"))
 (segment (start 5.511 60.978) (end 4.495 59.962) (width 0.2032) (layer "B.Cu") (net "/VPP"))
 (segment (start 7.02217 48.22) (end 7.585941 47.555005) (width 0.2032) (layer "B.Cu") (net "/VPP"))
 (segment (start 11.099 60.978) (end 5.511 60.978) (width 0.2032) (layer "B.Cu") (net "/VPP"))
 (segment (start 7.591 42.22) (end 9.091 40.72) (width 0.2032) (layer "B.Cu") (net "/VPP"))
 (segment (start 4.495 59.962) (end 4.495 50.74717) (width 0.2032) (layer "B.Cu") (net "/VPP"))
 (segment (start 17.253 29.558) (end 21.887 29.558) (width 0.254) (layer "B.Cu") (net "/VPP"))
 (segment (start 10.841 16.97) (end 11.341 16.47) (width 0.254) (layer "F.Cu") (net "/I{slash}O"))
 (segment (start 23.091 45.97) (end 23.091 46.72) (width 0.2032) (layer "F.Cu") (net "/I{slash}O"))
 (segment (start 8.341 24.22) (end 10.841 21.72) (width 0.254) (layer "F.Cu") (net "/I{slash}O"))
 (segment (start 13.341 16.47) (end 14.321 17.45) (width 0.254) (layer "F.Cu") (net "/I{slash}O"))
 (segment (start 14.321 17.45) (end 14.381 17.45) (width 0.254) (layer "F.Cu") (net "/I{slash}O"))
 (segment (start 18.341 51.47) (end 18.341 58.816) (width 0.2032) (layer "F.Cu") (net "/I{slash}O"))
 (segment (start 8.591 34.22) (end 6.091 31.72) (width 0.254) (layer "F.Cu") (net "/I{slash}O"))
 (segment (start 6.091 24.22) (end 8.341 24.22) (width 0.254) (layer "F.Cu") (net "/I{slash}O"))
 (segment (start 11.341 16.47) (end 13.341 16.47) (width 0.254) (layer "F.Cu") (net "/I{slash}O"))
 (segment (start 10.841 21.72) (end 10.841 16.97) (width 0.254) (layer "F.Cu") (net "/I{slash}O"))
 (segment (start 9.701 34.24) (end 8.611 34.24) (width 0.254) (layer "F.Cu") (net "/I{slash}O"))
 (segment (start 15.771 61.386) (end 14.655 61.386) (width 0.2032) (layer "F.Cu") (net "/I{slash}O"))
 (segment (start 6.091 31.72) (end 6.091 24.22) (width 0.254) (layer "F.Cu") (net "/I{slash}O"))
 (segment (start 23.091 46.72) (end 18.341 51.47) (width 0.2032) (layer "F.Cu") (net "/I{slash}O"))
 (segment (start 18.341 58.816) (end 15.771 61.386) (width 0.2032) (layer "F.Cu") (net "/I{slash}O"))
 (via (at 23.091 45.97) (size 0.6548) (drill 0.35) (layers "F.Cu" "B.Cu") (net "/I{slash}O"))
 (via (at 8.591 34.22) (size 0.6548) (drill 0.35) (layers "F.Cu" "B.Cu") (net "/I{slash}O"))
 (segment (start 23.091 42.72) (end 23.091 32.97) (width 0.254) (layer "B.Cu") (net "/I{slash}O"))
 (segment (start 8.591 34.22) (end 15.841 34.22) (width 0.254) (layer "B.Cu") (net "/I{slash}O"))
 (segment (start 23.091 32.97) (end 22.219 32.098) (width 0.254) (layer "B.Cu") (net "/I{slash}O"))
 (segment (start 23.091 45.97) (end 23.091 42.72) (width 0.2032) (layer "B.Cu") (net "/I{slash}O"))
 (segment (start 17.963 32.098) (end 21.887 32.098) (width 0.254) (layer "B.Cu") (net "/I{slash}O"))
 (segment (start 22.219 32.098) (end 21.887 32.098) (width 0.254) (layer "B.Cu") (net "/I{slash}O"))
 (segment (start 15.841 34.22) (end 17.963 32.098) (width 0.254) (layer "B.Cu") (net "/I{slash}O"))
 (segment (start 8.651 36.78) (end 8.591 36.72) (width 0.254) (layer "F.Cu") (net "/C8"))
 (segment (start 9.701 36.78) (end 8.651 36.78) (width 0.254) (layer "F.Cu") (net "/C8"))
 (via (at 8.591 36.72) (size 0.6548) (drill 0.35) (layers "F.Cu" "B.Cu") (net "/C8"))
 (segment (start 16.591 36.72) (end 18.673 34.638) (width 0.254) (layer "B.Cu") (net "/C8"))
 (segment (start 18.673 34.638) (end 21.887 34.638) (width 0.254) (layer "B.Cu") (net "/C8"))
 (segment (start 4.591 33.47) (end 7.841 36.72) (width 0.254) (layer "B.Cu") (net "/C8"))
 (segment (start 7.841 36.72) (end 8.591 36.72) (width 0.254) (layer "B.Cu") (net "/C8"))
 (segment (start 8.591 36.72) (end 16.591 36.72) (width 0.254) (layer "B.Cu") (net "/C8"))
 (segment (start 17.226 15.105) (end 17.226 13.97) (width 0.6096) (layer "F.Cu") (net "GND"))
 (segment (start 14.216 38.97) (end 14.216 26.845) (width 0.6096) (layer "F.Cu") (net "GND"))
 (segment (start 12.101 39.095) (end 14.841 39.095) (width 0.6096) (layer "F.Cu") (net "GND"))
 (segment (start 5.891 54.92) (end 5.891 54.452756) (width 0.6096) (layer "F.Cu") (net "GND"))
 (segment (start 14.341 39.095) (end 14.216 38.97) (width 0.6096) (layer "F.Cu") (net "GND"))
 (segment (start 6.456 13.835) (end 6.591 13.97) (width 0.6096) (layer "F.Cu") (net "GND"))
 (segment (start 20.751 56.01) (end 20.925 55.836) (width 0.6096) (layer "F.Cu") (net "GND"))
 (segment (start 20.925 55.836) (end 20.925 54.500591) (width 0.6096) (layer "F.Cu") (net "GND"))
 (segment (start 19.341 17.22) (end 17.226 15.105) (width 0.6096) (layer "F.Cu") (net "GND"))
 (segment (start 17.226 13.97) (end 17.226 11.47) (width 0.6096) (layer "F.Cu") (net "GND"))
 (segment (start 10.341 39.72) (end 11.476 39.72) (width 0.6096) (layer "F.Cu") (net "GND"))
 (segment (start 20.925 54.469577) (end 20.925 53.136) (width 0.6096) (layer "F.Cu") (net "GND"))
 (segment (start 6.456 11.47) (end 6.456 13.835) (width 0.6096) (layer "F.Cu") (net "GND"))
 (segment (start 11.476 39.72) (end 12.101 39.095) (width 0.6096) (layer "F.Cu") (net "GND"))
 (segment (start 14.216 26.845) (end 20.301 26.845) (width 0.6096) (layer "F.Cu") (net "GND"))
 (segment (start 18.966 26.845) (end 19.341 26.47) (width 0.6096) (layer "F.Cu") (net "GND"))
 (segment (start 19.341 26.47) (end 19.341 17.22) (width 0.6096) (layer "F.Cu") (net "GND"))
 (segment (start 5.891 54.446864) (end 5.891 52.12) (width 0.6096) (layer "F.Cu") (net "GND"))
 (segment (start 14.216 26.845) (end 12.101 26.845) (width 0.6096) (layer "F.Cu") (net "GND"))
 (segment (start 20.301 26.845) (end 18.966 26.845) (width 0.6096) (layer "F.Cu") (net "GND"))
 (segment (start 14.841 39.095) (end 20.301 39.095) (width 0.6096) (layer "F.Cu") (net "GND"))
 (via (at 6.591 13.97) (size 0.6548) (drill 0.35) (layers "F.Cu" "B.Cu") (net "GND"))
 (via (at 5.888054 54.44981) (size 0.6548) (drill 0.35) (layers "F.Cu" "B.Cu") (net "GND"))
 (via (at 20.909493 54.485084) (size 0.6548) (drill 0.35) (layers "F.Cu" "B.Cu") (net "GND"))
 (via (at 17.226 13.97) (size 0.6548) (drill 0.35) (layers "F.Cu" "B.Cu") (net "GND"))
 (segment (start 5.915621 54.491161) (end 6.520923 54.491161) (width 0.6096) (layer "B.Cu") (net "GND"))
 (segment (start 20.909493 54.485084) (end 6.527 54.485084) (width 0.6096) (layer "B.Cu") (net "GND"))
 (segment (start 6.591 13.97) (end 17.226 13.97) (width 0.6096) (layer "B.Cu") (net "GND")))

